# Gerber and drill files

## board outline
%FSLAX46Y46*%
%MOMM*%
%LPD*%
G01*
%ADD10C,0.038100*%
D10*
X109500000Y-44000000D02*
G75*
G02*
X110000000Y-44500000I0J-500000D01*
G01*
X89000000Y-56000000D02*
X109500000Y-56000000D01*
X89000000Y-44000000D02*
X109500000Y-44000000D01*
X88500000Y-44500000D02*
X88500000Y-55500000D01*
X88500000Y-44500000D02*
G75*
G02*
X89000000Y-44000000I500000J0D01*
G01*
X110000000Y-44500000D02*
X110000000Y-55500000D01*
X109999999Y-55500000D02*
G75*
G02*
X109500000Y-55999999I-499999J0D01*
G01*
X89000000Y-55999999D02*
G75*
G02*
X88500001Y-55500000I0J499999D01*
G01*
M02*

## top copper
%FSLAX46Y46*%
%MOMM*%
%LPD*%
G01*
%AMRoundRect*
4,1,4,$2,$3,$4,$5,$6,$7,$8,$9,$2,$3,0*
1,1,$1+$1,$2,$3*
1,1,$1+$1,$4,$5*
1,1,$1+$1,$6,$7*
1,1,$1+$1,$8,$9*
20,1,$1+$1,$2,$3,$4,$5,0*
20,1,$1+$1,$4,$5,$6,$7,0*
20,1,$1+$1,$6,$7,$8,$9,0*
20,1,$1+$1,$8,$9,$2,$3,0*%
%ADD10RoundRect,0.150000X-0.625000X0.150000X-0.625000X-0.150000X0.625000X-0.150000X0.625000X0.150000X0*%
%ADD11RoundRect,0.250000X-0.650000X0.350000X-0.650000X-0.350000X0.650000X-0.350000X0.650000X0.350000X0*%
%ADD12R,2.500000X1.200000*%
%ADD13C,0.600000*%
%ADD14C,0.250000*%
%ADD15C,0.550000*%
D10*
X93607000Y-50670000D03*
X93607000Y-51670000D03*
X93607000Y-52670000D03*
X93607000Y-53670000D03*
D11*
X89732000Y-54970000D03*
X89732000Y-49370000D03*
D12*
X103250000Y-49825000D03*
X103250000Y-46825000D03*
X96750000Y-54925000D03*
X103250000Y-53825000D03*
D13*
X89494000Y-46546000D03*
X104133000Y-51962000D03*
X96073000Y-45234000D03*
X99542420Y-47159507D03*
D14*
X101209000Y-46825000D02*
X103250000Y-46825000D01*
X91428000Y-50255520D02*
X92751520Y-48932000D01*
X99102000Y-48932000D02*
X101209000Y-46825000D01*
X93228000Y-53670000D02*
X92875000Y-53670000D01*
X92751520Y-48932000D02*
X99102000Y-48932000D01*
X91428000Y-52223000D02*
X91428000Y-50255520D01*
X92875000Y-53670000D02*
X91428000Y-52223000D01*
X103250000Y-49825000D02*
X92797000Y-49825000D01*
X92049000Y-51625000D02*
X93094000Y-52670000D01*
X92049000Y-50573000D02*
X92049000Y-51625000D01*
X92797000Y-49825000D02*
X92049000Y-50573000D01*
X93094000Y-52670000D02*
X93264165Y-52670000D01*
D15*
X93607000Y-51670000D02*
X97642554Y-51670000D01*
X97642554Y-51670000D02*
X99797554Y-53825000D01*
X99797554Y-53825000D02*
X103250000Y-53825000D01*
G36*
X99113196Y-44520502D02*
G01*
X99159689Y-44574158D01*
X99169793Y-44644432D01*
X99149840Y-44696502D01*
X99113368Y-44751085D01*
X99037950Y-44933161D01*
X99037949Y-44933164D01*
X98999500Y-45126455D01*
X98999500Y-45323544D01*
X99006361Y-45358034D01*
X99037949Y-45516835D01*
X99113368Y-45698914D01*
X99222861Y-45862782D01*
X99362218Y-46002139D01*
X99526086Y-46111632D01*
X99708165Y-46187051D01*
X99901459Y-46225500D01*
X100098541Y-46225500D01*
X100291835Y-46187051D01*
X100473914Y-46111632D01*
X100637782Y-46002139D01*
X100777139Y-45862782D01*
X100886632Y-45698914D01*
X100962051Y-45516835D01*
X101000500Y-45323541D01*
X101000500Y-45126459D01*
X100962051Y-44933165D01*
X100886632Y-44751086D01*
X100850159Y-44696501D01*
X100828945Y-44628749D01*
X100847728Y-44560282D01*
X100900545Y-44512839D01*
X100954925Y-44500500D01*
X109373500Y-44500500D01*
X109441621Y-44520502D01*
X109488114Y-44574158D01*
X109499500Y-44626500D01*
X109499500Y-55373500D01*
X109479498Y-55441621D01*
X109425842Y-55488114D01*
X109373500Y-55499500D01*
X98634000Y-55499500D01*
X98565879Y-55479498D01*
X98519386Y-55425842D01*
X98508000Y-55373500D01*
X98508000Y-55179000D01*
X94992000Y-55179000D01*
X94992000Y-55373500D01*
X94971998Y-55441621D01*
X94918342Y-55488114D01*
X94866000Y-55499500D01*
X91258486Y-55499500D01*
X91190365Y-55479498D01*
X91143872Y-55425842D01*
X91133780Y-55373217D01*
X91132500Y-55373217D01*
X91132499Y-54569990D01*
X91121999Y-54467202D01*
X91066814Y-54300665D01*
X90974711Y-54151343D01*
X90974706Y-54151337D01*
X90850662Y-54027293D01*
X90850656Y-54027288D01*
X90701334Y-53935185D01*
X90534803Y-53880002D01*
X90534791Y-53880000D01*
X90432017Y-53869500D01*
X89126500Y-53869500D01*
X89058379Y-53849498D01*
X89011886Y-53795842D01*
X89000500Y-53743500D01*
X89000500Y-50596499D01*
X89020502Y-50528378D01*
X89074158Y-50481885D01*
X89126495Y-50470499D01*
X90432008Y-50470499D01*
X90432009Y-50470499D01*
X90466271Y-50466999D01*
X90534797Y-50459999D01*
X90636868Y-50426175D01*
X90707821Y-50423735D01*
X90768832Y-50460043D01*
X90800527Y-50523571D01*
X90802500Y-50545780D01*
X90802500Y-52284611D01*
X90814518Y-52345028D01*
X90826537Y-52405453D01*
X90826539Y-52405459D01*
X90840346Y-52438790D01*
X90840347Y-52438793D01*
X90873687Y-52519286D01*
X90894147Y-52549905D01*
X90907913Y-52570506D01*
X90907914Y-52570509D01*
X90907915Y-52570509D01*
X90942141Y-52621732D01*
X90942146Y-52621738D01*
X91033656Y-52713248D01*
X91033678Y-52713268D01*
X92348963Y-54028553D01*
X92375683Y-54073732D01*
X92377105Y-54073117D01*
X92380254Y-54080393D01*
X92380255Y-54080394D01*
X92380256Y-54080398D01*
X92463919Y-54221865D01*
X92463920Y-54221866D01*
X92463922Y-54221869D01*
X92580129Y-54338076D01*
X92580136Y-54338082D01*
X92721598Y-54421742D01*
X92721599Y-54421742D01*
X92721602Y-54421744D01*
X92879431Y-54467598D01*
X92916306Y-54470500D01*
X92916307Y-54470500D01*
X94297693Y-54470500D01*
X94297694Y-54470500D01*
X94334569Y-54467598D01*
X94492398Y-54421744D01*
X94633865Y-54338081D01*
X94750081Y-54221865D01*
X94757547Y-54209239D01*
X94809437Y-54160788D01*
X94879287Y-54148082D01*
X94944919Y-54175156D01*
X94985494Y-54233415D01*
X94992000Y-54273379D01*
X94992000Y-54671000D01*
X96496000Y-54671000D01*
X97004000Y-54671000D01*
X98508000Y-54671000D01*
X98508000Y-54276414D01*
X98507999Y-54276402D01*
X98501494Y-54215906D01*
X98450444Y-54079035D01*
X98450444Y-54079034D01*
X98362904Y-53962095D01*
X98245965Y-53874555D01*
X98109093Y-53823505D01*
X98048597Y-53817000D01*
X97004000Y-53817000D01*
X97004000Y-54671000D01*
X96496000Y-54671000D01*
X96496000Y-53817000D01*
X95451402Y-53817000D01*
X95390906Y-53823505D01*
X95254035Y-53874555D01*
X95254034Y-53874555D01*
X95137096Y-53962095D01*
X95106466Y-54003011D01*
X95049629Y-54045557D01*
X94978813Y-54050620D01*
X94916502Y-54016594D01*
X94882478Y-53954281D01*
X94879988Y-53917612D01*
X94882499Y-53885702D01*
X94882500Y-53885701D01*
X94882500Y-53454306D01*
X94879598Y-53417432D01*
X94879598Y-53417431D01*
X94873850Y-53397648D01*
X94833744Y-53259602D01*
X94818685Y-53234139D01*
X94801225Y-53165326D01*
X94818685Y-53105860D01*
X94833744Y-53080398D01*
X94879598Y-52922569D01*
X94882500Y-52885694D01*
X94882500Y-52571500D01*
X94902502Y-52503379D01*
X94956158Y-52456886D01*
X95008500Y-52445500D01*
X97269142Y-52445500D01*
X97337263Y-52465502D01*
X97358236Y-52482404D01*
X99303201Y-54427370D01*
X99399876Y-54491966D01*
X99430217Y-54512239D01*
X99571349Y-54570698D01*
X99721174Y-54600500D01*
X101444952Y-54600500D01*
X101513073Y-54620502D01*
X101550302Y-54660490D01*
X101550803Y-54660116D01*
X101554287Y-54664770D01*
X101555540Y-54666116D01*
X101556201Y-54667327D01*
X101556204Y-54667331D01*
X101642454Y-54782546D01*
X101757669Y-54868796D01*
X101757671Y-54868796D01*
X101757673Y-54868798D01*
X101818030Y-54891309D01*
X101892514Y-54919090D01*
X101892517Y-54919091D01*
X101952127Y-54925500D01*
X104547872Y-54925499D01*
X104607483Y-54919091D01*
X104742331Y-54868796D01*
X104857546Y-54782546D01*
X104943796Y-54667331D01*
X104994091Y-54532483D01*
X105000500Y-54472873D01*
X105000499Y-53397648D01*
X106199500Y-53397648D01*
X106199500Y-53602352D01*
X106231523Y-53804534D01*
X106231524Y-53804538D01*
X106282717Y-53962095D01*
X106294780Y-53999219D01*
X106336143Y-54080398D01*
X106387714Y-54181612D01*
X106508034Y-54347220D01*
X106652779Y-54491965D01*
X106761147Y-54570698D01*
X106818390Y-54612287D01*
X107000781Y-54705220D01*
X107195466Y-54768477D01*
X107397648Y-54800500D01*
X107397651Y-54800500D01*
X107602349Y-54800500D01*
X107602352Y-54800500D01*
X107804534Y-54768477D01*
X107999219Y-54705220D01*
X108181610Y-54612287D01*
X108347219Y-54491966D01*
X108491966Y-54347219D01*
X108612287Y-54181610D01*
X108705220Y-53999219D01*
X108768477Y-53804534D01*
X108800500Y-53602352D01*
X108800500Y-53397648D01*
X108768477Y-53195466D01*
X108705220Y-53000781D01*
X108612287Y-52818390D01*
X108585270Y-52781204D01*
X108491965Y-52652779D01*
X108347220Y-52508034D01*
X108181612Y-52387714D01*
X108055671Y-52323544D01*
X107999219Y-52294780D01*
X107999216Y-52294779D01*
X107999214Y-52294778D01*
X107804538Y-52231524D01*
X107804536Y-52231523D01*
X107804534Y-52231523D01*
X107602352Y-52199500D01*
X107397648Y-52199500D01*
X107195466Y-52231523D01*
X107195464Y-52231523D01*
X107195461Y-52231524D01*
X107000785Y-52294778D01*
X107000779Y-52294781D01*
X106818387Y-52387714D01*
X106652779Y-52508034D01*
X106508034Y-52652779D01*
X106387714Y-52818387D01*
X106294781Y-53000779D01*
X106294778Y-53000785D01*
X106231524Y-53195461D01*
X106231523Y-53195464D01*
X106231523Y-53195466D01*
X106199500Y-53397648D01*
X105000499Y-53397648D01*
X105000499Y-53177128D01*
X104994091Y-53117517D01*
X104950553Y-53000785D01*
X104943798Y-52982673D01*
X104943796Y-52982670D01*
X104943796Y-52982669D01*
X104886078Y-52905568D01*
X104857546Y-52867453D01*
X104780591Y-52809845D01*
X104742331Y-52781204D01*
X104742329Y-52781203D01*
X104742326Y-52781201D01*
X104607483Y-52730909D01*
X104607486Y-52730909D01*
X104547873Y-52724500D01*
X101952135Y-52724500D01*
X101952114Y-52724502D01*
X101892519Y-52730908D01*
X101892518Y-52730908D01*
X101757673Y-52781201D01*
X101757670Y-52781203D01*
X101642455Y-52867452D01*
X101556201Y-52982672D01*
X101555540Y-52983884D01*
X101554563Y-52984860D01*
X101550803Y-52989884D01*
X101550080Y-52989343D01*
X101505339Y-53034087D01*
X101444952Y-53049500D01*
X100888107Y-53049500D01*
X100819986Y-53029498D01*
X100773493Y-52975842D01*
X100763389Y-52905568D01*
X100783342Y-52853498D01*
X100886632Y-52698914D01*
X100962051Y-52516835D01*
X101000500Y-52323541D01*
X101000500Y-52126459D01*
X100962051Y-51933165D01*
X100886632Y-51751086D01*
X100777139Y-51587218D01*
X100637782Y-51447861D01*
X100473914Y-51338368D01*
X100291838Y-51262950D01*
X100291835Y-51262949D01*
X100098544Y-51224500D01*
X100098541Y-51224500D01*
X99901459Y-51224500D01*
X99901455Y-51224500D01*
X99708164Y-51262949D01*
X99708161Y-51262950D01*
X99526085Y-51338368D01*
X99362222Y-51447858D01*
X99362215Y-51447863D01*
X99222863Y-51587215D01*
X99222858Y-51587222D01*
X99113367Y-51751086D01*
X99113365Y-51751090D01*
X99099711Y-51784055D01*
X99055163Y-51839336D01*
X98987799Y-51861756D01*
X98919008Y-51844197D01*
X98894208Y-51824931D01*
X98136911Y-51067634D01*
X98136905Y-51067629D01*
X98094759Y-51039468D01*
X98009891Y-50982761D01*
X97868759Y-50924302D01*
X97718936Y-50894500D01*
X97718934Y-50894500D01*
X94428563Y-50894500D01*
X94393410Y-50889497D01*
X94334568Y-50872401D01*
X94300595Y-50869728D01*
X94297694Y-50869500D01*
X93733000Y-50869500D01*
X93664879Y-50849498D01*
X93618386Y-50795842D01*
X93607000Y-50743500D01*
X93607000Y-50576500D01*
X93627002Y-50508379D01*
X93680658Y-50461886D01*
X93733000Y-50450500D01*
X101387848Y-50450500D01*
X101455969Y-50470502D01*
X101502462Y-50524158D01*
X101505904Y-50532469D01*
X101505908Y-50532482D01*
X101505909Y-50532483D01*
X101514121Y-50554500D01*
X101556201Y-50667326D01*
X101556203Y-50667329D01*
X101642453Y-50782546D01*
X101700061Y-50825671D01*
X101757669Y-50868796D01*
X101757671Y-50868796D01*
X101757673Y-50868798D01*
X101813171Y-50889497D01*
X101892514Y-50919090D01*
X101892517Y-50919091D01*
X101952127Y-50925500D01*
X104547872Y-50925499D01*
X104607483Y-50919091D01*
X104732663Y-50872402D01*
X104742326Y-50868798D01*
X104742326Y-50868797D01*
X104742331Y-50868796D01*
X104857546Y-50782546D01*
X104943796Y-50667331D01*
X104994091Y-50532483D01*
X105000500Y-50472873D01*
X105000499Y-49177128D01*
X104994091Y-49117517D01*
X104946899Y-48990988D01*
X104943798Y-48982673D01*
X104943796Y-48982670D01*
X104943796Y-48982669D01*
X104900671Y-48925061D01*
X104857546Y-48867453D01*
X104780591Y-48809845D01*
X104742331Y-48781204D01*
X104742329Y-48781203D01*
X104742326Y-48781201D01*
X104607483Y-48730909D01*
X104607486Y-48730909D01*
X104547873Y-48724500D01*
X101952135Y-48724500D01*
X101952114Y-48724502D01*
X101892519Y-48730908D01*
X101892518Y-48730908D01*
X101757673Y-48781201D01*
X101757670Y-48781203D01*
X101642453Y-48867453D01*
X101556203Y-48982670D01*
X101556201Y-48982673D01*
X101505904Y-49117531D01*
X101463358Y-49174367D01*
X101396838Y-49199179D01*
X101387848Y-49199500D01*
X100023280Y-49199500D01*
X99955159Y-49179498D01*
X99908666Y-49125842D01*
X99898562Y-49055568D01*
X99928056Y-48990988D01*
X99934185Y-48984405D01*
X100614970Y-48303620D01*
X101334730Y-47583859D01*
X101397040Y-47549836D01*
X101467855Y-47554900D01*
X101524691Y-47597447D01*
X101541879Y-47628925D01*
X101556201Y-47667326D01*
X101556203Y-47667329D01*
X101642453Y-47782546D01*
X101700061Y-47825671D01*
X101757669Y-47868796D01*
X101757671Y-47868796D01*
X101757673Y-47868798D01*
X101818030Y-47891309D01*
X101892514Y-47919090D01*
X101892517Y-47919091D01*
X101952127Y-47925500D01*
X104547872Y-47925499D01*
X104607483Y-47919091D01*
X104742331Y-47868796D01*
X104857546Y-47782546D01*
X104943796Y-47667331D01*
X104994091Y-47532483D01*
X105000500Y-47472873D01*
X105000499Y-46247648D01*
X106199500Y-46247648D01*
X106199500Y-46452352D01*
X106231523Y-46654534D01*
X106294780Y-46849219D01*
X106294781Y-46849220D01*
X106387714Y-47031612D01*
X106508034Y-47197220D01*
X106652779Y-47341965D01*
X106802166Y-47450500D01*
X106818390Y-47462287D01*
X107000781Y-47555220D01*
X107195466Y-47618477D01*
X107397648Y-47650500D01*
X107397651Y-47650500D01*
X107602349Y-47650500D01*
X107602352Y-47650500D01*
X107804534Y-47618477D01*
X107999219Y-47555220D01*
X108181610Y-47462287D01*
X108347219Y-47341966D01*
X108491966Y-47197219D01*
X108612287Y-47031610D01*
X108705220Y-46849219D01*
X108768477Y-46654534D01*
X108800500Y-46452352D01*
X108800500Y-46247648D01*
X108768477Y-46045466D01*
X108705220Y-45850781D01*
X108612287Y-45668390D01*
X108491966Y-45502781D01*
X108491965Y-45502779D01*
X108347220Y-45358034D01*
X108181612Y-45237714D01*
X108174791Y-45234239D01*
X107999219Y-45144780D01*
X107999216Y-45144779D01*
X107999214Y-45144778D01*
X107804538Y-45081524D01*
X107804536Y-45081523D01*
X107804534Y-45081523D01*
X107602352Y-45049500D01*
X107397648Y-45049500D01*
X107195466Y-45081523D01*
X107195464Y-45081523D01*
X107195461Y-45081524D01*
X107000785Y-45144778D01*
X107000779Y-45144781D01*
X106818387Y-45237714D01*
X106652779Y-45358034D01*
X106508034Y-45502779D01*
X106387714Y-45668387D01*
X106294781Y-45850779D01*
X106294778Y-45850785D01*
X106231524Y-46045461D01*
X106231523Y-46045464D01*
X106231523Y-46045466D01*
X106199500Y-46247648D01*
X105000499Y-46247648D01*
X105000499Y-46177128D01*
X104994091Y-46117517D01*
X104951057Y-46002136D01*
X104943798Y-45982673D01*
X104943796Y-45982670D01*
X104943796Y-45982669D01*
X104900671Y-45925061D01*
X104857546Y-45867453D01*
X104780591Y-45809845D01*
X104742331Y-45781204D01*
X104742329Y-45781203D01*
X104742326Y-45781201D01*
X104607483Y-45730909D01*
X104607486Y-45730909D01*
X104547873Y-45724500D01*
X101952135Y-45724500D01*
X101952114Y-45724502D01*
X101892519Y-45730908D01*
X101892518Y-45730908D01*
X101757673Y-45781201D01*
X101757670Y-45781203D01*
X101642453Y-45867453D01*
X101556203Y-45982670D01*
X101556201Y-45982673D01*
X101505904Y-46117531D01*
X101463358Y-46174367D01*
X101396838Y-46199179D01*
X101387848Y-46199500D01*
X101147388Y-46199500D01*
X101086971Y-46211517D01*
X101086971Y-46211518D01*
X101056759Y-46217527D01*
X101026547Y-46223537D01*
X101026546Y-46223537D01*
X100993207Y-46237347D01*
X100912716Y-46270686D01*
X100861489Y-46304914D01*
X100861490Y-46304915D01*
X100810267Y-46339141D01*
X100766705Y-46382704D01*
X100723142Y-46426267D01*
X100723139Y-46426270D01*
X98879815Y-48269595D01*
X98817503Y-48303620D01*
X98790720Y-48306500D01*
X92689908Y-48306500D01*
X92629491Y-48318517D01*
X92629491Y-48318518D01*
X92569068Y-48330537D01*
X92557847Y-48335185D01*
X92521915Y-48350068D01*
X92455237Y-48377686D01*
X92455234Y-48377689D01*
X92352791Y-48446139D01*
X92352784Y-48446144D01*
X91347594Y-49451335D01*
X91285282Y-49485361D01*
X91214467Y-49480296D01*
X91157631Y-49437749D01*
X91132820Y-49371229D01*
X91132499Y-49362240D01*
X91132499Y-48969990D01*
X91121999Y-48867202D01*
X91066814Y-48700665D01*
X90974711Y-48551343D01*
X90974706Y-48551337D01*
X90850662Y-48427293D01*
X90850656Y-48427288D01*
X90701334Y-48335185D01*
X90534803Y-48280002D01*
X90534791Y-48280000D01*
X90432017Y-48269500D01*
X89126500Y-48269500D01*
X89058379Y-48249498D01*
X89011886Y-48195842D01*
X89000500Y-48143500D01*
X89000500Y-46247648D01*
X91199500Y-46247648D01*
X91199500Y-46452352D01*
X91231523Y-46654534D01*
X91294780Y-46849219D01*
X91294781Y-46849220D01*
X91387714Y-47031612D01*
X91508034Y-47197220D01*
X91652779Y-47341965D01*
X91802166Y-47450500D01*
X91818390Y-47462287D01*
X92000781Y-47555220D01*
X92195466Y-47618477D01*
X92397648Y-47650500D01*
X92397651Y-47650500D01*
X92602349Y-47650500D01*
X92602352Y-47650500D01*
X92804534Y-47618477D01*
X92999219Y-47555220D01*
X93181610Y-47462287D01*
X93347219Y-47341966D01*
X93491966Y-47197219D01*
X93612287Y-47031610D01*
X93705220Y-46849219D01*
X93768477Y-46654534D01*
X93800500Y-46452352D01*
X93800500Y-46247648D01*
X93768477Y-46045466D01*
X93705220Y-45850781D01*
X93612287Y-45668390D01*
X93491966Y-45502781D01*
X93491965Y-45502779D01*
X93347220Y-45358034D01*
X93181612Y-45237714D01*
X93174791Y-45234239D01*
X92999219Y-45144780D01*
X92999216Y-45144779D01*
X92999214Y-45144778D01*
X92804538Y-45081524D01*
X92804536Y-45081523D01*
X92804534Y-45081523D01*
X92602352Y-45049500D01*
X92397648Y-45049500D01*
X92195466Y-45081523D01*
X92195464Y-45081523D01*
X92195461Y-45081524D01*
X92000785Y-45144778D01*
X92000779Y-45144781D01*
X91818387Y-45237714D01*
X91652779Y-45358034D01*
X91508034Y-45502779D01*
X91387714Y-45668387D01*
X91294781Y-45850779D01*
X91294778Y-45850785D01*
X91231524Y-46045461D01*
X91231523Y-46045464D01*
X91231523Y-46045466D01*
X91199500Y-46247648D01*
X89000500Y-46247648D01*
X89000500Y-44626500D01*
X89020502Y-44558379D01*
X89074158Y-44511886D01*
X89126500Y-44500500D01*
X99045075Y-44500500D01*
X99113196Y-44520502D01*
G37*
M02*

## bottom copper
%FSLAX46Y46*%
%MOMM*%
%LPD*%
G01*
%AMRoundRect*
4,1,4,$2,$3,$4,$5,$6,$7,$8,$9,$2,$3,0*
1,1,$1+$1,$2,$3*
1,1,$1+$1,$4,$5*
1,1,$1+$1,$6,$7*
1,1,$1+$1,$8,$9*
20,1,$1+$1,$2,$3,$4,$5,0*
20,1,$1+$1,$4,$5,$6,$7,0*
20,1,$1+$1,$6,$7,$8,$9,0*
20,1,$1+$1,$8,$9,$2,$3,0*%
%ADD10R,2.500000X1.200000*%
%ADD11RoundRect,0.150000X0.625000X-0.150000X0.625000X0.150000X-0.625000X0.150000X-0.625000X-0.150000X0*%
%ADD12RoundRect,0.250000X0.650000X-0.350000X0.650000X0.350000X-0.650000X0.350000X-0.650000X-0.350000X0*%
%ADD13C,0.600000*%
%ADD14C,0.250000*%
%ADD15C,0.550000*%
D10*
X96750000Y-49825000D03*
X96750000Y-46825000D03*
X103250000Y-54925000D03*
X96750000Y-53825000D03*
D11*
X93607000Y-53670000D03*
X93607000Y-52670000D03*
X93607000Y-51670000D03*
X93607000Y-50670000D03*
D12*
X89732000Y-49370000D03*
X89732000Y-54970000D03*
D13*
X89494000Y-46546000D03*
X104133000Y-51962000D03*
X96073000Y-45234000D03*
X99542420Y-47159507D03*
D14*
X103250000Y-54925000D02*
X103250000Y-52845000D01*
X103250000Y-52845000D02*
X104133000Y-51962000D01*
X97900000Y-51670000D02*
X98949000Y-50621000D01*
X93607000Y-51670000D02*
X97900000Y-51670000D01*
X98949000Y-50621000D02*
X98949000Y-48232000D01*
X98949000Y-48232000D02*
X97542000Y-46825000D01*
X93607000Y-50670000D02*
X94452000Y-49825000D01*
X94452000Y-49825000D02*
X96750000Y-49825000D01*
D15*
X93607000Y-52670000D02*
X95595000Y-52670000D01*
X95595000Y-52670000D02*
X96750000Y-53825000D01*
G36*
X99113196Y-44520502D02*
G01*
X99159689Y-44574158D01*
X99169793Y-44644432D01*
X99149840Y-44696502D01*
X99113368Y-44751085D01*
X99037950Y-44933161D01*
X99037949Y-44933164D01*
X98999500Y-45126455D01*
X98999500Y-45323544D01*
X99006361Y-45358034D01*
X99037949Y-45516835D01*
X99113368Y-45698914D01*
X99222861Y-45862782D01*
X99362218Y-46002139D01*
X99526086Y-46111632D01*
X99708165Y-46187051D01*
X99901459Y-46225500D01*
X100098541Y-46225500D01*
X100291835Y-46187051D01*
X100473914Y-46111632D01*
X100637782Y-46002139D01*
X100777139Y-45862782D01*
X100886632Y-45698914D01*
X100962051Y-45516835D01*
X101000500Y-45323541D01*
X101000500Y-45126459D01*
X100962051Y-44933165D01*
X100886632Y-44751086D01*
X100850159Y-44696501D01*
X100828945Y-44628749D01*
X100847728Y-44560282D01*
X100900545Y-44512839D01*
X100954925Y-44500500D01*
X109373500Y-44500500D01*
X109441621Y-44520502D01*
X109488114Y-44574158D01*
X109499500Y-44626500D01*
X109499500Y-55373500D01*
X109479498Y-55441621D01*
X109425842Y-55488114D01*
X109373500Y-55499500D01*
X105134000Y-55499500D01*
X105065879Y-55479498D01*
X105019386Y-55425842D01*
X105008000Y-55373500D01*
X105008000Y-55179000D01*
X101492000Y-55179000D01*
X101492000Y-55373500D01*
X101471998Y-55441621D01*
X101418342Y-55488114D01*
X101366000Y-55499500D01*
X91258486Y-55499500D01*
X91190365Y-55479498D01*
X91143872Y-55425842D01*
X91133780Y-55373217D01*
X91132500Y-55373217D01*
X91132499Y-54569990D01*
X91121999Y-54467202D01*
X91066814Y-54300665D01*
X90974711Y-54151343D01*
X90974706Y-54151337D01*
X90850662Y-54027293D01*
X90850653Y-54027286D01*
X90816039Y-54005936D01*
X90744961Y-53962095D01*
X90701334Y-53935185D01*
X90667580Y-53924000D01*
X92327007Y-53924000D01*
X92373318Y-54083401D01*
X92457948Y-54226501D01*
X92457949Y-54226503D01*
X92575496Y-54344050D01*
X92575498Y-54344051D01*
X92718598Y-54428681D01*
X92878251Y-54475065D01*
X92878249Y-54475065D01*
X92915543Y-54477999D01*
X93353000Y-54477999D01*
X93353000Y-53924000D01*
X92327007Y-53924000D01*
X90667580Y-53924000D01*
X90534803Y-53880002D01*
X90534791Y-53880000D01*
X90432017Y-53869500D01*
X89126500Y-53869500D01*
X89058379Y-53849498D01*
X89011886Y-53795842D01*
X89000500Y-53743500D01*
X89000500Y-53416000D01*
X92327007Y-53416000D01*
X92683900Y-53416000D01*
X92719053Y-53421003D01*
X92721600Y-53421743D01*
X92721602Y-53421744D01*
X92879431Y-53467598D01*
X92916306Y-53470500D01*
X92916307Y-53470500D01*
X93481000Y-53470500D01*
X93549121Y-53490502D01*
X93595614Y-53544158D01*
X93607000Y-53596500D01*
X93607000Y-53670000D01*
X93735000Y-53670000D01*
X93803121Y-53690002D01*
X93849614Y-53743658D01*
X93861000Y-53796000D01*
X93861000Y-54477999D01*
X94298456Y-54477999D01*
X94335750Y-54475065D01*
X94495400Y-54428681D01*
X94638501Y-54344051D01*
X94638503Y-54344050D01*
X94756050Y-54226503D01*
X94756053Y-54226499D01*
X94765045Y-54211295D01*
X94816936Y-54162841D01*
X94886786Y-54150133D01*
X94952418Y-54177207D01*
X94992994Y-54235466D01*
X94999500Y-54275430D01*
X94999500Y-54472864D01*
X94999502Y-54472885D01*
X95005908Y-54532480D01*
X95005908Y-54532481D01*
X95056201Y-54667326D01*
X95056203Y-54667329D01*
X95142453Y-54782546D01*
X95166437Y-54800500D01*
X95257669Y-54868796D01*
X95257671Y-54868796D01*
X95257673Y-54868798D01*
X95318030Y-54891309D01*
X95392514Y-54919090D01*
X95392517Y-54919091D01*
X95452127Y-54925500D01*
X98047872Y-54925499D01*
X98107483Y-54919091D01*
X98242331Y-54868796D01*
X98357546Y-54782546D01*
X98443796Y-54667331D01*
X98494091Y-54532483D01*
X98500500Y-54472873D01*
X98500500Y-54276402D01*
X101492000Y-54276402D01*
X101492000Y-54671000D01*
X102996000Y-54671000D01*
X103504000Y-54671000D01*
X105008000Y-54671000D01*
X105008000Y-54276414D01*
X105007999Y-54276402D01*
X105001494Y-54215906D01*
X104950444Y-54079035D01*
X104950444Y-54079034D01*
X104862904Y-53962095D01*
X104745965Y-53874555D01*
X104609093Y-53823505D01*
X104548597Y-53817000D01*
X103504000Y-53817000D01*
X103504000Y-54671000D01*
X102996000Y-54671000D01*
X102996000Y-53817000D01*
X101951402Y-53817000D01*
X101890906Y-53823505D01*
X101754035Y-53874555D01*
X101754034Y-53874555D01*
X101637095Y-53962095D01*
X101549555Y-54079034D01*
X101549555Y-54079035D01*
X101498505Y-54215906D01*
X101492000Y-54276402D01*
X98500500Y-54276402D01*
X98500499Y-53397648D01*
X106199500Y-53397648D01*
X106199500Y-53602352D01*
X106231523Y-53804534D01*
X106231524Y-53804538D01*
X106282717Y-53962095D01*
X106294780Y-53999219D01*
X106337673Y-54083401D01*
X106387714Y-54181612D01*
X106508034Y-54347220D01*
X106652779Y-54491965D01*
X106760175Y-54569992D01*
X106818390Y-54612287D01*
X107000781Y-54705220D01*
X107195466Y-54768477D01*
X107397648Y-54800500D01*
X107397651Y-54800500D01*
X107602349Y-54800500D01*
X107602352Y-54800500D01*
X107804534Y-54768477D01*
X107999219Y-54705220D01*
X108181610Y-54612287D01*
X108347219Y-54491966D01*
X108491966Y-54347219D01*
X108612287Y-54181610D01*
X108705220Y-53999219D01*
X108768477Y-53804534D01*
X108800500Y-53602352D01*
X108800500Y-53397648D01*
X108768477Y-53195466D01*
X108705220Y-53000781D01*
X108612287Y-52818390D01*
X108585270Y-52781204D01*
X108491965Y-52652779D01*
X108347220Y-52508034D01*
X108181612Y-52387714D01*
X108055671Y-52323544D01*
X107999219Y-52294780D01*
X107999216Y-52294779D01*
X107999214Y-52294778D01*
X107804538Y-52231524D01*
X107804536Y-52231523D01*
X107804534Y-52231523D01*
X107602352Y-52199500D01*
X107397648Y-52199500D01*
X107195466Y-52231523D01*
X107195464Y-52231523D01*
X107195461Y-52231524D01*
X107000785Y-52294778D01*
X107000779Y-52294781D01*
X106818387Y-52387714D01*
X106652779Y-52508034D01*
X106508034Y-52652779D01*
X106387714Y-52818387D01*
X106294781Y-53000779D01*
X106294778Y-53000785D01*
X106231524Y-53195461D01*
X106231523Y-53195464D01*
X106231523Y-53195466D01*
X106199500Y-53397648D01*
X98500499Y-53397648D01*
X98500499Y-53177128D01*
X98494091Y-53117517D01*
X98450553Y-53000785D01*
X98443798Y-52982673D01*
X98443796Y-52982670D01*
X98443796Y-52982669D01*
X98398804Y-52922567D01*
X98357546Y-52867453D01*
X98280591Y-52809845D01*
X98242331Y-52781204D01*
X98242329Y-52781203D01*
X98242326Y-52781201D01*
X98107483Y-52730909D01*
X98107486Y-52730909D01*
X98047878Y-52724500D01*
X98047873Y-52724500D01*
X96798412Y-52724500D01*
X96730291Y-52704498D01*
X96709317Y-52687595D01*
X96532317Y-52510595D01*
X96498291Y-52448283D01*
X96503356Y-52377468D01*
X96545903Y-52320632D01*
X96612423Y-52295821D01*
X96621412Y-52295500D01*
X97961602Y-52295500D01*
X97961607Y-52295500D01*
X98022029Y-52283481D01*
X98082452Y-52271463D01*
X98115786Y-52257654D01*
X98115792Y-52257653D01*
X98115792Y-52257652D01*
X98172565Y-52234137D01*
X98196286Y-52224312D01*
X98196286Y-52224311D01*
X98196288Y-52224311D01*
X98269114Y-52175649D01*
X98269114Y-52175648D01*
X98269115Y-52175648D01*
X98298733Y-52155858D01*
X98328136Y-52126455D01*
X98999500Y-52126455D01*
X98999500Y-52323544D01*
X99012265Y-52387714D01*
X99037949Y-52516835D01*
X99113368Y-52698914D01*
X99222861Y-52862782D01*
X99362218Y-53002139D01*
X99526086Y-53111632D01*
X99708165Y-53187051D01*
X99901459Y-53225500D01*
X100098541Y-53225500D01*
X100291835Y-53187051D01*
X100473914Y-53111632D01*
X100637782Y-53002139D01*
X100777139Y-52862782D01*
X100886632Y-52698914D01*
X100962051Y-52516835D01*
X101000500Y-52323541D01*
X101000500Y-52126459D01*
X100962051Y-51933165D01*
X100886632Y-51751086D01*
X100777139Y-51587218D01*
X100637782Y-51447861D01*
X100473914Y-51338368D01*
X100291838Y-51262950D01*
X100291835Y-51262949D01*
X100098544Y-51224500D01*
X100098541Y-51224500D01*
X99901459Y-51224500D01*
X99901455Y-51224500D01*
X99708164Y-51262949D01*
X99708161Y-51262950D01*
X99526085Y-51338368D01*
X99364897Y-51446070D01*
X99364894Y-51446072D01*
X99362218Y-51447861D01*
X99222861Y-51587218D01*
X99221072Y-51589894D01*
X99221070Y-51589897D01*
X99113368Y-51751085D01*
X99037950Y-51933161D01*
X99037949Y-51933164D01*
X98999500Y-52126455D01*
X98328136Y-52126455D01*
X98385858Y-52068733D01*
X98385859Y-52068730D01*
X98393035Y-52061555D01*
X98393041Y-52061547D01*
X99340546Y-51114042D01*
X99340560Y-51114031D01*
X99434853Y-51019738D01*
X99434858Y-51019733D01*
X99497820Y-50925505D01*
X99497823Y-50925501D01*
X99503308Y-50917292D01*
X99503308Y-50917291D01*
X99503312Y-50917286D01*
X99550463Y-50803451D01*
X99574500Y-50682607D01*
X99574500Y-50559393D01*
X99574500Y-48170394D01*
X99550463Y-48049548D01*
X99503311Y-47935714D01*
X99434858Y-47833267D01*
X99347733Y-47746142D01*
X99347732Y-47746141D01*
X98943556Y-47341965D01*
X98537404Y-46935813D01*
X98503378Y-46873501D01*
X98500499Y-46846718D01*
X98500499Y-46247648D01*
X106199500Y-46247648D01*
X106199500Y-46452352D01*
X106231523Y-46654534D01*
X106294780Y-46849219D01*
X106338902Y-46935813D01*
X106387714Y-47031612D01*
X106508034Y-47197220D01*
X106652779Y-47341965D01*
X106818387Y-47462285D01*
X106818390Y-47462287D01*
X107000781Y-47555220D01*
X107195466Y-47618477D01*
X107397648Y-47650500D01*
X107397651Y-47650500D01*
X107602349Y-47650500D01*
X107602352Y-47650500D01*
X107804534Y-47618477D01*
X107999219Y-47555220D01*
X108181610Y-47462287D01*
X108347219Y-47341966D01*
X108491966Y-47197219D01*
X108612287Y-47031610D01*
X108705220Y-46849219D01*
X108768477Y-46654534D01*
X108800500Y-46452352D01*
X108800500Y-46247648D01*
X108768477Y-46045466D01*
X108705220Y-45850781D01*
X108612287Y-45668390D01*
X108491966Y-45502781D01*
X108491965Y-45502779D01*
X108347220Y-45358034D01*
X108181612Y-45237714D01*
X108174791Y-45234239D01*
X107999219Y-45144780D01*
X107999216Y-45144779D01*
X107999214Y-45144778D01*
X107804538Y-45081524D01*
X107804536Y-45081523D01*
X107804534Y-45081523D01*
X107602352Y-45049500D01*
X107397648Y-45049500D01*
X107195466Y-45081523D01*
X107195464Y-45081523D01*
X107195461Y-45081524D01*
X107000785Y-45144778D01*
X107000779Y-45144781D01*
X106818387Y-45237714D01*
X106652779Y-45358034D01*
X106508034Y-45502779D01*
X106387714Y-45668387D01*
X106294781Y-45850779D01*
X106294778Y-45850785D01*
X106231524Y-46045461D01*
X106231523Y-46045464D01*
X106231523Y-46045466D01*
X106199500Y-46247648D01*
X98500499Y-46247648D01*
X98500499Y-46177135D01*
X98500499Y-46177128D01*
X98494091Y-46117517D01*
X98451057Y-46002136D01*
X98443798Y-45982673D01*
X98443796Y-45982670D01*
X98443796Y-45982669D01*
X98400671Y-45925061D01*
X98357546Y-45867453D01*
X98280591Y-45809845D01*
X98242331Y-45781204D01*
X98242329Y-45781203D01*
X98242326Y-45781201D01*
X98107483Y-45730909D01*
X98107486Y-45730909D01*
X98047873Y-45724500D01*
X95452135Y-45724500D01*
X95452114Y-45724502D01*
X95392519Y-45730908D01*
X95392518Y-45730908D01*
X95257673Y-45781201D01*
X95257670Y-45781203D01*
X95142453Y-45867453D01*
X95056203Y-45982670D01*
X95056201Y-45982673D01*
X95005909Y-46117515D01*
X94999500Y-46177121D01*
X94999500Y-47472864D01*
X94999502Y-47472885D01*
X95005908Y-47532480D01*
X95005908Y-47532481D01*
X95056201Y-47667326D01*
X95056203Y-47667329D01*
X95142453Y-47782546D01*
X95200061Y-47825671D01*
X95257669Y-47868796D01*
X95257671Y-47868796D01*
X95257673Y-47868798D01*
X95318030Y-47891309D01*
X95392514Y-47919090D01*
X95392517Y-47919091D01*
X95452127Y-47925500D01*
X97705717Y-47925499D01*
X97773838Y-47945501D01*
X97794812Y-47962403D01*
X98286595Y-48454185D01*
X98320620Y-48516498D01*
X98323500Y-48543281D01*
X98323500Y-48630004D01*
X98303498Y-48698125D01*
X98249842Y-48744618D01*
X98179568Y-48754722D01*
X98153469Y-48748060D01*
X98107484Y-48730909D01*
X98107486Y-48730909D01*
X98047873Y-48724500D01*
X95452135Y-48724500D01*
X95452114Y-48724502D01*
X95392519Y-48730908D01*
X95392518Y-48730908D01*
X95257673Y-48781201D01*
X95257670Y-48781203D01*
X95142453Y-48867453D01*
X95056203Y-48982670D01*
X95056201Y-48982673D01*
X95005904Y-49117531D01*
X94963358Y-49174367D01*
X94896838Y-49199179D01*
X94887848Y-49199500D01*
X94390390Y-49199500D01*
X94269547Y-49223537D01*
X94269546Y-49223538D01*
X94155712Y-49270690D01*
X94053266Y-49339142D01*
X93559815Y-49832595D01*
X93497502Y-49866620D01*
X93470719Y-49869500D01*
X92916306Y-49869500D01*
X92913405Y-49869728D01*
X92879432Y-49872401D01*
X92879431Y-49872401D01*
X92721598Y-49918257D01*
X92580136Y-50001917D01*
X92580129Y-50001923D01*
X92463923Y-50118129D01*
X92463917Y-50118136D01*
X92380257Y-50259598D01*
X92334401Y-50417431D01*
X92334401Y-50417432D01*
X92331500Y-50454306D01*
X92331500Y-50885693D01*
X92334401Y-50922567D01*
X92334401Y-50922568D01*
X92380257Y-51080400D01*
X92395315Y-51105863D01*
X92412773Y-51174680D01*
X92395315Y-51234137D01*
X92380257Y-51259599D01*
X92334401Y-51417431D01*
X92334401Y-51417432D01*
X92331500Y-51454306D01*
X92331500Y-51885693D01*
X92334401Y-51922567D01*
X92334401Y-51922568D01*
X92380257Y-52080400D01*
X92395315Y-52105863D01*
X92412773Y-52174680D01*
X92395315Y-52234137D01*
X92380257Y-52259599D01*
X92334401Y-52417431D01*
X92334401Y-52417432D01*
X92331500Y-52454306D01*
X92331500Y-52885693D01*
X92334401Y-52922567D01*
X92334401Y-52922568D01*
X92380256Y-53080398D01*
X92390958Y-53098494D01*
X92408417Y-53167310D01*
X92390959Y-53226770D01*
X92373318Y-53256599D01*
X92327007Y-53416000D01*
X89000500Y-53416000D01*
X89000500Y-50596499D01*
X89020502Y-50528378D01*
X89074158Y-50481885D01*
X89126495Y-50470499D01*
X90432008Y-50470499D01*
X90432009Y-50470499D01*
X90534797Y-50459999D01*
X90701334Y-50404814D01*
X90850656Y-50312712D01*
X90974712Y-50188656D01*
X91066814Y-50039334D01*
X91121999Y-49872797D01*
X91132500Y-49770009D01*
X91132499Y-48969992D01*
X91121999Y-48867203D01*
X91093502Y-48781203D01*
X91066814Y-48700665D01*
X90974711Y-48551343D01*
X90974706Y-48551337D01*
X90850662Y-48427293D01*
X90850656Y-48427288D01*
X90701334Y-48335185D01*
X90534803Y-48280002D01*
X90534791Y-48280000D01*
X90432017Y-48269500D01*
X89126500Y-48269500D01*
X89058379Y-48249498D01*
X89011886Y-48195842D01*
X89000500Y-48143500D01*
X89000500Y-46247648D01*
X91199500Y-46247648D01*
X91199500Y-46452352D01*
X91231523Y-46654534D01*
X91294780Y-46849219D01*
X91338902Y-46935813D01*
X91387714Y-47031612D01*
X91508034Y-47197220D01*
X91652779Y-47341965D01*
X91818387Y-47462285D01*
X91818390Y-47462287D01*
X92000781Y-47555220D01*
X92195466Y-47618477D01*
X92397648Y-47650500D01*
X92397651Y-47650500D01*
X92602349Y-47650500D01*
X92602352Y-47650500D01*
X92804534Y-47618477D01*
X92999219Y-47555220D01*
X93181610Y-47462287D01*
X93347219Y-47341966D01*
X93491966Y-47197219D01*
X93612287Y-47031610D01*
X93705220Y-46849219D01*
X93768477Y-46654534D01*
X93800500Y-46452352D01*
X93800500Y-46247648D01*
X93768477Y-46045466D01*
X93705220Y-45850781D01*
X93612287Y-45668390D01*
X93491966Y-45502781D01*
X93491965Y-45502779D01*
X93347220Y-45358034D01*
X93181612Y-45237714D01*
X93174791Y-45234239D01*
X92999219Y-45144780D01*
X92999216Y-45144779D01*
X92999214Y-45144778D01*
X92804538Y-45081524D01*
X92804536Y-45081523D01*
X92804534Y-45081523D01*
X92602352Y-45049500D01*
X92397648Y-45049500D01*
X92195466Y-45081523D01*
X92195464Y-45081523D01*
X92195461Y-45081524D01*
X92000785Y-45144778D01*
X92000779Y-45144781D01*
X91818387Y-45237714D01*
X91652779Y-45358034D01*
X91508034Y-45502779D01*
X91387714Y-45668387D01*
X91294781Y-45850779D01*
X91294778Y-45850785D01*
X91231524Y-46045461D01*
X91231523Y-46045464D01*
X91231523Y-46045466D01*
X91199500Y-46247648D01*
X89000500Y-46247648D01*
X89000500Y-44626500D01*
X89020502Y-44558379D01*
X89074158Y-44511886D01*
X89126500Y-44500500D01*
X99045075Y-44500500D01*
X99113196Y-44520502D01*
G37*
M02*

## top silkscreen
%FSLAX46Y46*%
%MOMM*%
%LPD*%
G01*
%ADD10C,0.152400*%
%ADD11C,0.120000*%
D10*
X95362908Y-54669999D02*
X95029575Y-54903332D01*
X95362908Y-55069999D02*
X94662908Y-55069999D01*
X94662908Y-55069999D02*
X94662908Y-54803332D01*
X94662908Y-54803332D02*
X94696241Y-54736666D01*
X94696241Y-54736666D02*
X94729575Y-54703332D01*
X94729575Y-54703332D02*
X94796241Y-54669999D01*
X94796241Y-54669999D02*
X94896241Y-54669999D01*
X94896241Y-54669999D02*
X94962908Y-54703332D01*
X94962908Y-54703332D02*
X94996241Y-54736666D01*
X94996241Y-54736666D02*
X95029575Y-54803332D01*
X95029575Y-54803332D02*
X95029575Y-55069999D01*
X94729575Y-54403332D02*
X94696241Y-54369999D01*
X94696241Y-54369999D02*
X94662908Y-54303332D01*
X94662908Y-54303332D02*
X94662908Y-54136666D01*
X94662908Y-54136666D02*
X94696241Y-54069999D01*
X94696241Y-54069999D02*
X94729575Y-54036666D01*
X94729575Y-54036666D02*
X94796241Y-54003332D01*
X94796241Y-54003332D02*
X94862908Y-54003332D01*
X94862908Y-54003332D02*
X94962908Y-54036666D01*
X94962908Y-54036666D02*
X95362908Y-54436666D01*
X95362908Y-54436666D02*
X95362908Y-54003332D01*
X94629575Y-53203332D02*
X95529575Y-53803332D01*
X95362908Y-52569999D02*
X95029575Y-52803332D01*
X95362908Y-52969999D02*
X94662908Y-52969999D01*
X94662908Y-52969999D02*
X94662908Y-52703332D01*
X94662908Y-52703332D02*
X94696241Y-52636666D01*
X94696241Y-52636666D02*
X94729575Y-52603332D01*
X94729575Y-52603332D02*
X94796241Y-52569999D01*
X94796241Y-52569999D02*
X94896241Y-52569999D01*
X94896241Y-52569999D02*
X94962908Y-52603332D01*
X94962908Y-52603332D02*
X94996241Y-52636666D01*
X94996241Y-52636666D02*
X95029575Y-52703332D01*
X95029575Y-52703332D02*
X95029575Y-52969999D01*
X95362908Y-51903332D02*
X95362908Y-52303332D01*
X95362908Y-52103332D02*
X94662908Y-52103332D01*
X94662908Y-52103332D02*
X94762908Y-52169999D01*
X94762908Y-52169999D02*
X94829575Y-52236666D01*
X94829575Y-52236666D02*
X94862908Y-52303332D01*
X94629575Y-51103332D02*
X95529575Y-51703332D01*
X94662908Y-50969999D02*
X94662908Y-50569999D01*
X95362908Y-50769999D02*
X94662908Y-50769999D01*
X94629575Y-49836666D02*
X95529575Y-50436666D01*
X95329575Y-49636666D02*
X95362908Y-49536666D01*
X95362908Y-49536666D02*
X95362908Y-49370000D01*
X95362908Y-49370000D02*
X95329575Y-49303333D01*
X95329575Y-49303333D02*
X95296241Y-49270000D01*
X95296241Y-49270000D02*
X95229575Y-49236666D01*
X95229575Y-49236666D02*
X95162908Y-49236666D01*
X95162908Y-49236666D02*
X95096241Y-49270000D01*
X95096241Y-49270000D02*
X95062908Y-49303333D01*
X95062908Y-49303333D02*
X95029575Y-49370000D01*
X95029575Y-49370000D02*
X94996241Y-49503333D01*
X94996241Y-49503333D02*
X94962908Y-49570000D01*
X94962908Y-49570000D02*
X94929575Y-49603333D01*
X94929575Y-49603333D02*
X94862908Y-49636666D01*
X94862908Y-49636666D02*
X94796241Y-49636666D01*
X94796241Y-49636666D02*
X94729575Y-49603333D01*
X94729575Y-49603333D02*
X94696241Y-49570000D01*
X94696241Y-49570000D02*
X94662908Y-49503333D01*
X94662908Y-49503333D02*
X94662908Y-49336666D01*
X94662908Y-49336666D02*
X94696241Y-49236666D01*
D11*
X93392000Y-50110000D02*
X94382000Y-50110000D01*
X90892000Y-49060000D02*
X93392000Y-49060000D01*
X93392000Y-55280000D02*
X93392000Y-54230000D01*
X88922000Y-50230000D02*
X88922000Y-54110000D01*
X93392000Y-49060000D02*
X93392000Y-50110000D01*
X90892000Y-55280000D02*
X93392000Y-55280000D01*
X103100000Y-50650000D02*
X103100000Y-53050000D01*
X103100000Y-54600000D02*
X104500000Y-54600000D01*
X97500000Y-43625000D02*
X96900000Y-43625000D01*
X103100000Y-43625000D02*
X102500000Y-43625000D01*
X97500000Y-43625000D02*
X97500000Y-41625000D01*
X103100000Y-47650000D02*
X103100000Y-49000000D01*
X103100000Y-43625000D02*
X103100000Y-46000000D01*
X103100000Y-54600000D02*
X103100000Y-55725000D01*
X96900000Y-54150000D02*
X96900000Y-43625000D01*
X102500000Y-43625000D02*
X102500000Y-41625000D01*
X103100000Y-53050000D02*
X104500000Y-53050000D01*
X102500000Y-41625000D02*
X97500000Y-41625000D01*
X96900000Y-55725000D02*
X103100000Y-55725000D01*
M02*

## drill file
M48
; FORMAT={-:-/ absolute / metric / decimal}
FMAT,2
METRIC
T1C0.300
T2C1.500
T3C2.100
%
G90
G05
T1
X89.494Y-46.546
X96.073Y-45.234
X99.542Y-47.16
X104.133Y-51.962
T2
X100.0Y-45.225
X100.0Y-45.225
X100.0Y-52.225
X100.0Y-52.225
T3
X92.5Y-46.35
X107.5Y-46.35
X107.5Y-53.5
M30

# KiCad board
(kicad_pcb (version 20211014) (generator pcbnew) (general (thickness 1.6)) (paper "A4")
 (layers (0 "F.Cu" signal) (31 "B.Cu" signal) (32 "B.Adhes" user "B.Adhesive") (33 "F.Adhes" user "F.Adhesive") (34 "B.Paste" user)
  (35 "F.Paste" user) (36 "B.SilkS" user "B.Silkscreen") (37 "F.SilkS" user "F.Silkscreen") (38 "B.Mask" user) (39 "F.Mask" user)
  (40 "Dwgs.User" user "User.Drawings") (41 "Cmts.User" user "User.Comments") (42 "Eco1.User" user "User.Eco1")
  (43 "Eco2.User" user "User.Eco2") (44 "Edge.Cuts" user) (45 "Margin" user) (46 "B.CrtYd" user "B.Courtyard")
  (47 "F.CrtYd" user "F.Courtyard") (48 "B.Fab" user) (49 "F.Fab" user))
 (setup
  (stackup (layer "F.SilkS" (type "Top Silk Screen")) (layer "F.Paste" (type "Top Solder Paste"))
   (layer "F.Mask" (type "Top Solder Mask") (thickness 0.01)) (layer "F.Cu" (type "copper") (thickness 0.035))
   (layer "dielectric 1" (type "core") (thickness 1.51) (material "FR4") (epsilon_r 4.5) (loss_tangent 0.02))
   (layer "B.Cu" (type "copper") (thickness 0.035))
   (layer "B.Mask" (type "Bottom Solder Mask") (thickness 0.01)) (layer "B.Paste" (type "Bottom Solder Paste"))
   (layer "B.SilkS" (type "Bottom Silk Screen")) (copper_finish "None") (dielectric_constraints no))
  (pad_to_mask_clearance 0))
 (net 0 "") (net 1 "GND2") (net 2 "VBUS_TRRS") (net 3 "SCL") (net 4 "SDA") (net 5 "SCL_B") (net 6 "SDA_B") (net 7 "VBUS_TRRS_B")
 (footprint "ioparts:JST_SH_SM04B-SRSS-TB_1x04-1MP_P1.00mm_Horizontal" (layer "F.Cu") (at 91.607 52.17 -90)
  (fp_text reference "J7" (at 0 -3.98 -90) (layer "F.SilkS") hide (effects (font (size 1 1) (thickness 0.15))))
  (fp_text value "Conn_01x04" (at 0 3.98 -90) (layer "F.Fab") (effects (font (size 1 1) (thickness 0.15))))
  (fp_line (start -2.06 -1.785) (end -2.06 -2.775) (layer "F.SilkS") (width 0.12))
  (fp_line (start -3.11 0.715) (end -3.11 -1.785) (layer "F.SilkS") (width 0.12))
  (fp_line (start 3.11 -1.785) (end 2.06 -1.785) (layer "F.SilkS") (width 0.12))
  (fp_line (start -1.94 2.685) (end 1.94 2.685) (layer "F.SilkS") (width 0.12))
  (fp_line (start -3.11 -1.785) (end -2.06 -1.785) (layer "F.SilkS") (width 0.12))
  (fp_line (start 3.11 0.715) (end 3.11 -1.785) (layer "F.SilkS") (width 0.12))
  (pad "1" smd roundrect (at -1.5 -2 270) (size 0.6 1.55) (layers "F.Cu" "F.Paste" "F.Mask") (roundrect_rratio 0.25) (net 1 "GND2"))
  (pad "2" smd roundrect (at -0.5 -2 270) (size 0.6 1.55) (layers "F.Cu" "F.Paste" "F.Mask") (roundrect_rratio 0.25) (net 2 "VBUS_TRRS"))
  (pad "3" smd roundrect (at 0.5 -2 270) (size 0.6 1.55) (layers "F.Cu" "F.Paste" "F.Mask") (roundrect_rratio 0.25) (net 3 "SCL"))
  (pad "4" smd roundrect (at 1.5 -2 270) (size 0.6 1.55) (layers "F.Cu" "F.Paste" "F.Mask") (roundrect_rratio 0.25) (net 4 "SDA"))
  (pad "MP" smd roundrect (at 2.8 1.875 270) (size 1.2 1.8) (layers "F.Cu" "F.Paste" "F.Mask") (roundrect_rratio 0.2083333333))
  (pad "MP" smd roundrect (at -2.8 1.875 270) (size 1.2 1.8) (layers "F.Cu" "F.Paste" "F.Mask") (roundrect_rratio 0.2083333333)))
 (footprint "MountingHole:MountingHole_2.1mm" (layer "F.Cu") (at 107.5 53.5)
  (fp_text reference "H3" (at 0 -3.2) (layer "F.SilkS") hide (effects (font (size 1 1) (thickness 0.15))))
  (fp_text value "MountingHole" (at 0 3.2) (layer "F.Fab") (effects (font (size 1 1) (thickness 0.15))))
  (pad "" np_thru_hole circle (at 0 0) (size 2.1 2.1) (drill 2.1) (layers *.Cu *.Mask)))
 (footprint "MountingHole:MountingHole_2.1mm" (layer "F.Cu") (at 92.5 46.35)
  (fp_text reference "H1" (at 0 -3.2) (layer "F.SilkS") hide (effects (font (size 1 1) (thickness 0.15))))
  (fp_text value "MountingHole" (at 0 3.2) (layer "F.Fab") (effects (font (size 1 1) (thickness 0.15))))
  (pad "" np_thru_hole circle (at 0 0) (size 2.1 2.1) (drill 2.1) (layers *.Cu *.Mask)))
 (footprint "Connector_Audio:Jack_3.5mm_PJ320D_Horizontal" (layer "F.Cu") (at 100 50 -90)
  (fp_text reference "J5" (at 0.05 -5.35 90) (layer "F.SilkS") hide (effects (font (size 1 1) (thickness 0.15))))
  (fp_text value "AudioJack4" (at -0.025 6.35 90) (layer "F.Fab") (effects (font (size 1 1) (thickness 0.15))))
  (fp_line (start 0.65 -3.1) (end 3.05 -3.1) (layer "F.SilkS") (width 0.12))
  (fp_line (start 4.6 -3.1) (end 4.6 -4.5) (layer "F.SilkS") (width 0.12))
  (fp_line (start -6.375 2.5) (end -6.375 3.1) (layer "F.SilkS") (width 0.12))
  (fp_line (start -6.375 -3.1) (end -6.375 -2.5) (layer "F.SilkS") (width 0.12))
  (fp_line (start -6.375 2.5) (end -8.375 2.5) (layer "F.SilkS") (width 0.12))
  (fp_line (start -2.35 -3.1) (end -1 -3.1) (layer "F.SilkS") (width 0.12))
  (fp_line (start -6.375 -3.1) (end -4 -3.1) (layer "F.SilkS") (width 0.12))
  (fp_line (start 4.6 -3.1) (end 5.725 -3.1) (layer "F.SilkS") (width 0.12))
  (fp_line (start 4.15 3.1) (end -6.375 3.1) (layer "F.SilkS") (width 0.12))
  (fp_line (start -6.375 -2.5) (end -8.375 -2.5) (layer "F.SilkS") (width 0.12))
  (fp_line (start 3.05 -3.1) (end 3.05 -4.5) (layer "F.SilkS") (width 0.12))
  (fp_line (start -8.375 -2.5) (end -8.375 2.5) (layer "F.SilkS") (width 0.12))
  (fp_line (start 5.725 3.1) (end 5.725 -3.1) (layer "F.SilkS") (width 0.12))
  (pad "" np_thru_hole circle (at -4.775 0 270) (size 1.5 1.5) (drill 1.5) (layers *.Cu *.Mask))
  (pad "" np_thru_hole circle (at 2.225 0 270) (size 1.5 1.5) (drill 1.5) (layers *.Cu *.Mask))
  (pad "R1" smd rect (at -0.175 -3.25 270) (size 1.2 2.5) (layers "F.Cu" "F.Paste" "F.Mask") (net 3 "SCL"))
  (pad "R2" smd rect (at -3.175 -3.25 270) (size 1.2 2.5) (layers "F.Cu" "F.Paste" "F.Mask") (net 4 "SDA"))
  (pad "S" smd rect (at 4.925 3.25 270) (size 1.2 2.5) (layers "F.Cu" "F.Paste" "F.Mask") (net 1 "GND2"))
  (pad "T" smd rect (at 3.825 -3.25 270) (size 1.2 2.5) (layers "F.Cu" "F.Paste" "F.Mask") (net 2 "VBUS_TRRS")))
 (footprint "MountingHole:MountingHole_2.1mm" (layer "F.Cu") (at 107.5 46.35)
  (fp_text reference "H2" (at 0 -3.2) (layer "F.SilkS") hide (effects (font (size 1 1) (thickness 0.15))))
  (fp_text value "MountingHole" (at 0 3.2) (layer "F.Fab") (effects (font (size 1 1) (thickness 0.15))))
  (pad "" np_thru_hole circle (at 0 0) (size 2.1 2.1) (drill 2.1) (layers *.Cu *.Mask)))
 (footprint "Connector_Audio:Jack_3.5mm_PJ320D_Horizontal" (layer "B.Cu") (at 100 50 -90)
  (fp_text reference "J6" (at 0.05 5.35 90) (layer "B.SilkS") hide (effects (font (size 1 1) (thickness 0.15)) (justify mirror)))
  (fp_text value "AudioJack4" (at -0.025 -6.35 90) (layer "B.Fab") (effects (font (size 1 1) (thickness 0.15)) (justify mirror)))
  (pad "" np_thru_hole circle (at 2.225 0 270) (size 1.5 1.5) (drill 1.5) (layers *.Cu *.Mask))
  (pad "" np_thru_hole circle (at -4.775 0 270) (size 1.5 1.5) (drill 1.5) (layers *.Cu *.Mask))
  (pad "R1" smd rect (at -0.175 3.25 270) (size 1.2 2.5) (layers "B.Cu" "B.Paste" "B.Mask") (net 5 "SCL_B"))
  (pad "R2" smd rect (at -3.175 3.25 270) (size 1.2 2.5) (layers "B.Cu" "B.Paste" "B.Mask") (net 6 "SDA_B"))
  (pad "S" smd rect (at 4.925 -3.25 270) (size 1.2 2.5) (layers "B.Cu" "B.Paste" "B.Mask") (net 1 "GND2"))
  (pad "T" smd rect (at 3.825 3.25 270) (size 1.2 2.5) (layers "B.Cu" "B.Paste" "B.Mask") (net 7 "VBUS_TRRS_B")))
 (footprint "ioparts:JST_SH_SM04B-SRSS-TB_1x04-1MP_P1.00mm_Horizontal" (layer "B.Cu") (at 91.607 52.17 90)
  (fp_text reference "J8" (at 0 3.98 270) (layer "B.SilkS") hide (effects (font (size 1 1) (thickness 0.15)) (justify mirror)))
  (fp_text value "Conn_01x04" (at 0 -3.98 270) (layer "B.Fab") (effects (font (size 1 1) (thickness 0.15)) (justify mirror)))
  (pad "1" smd roundrect (at -1.5 2 90) (size 0.6 1.55) (layers "B.Cu" "B.Paste" "B.Mask") (roundrect_rratio 0.25) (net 1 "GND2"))
  (pad "2" smd roundrect (at -0.5 2 90) (size 0.6 1.55) (layers "B.Cu" "B.Paste" "B.Mask") (roundrect_rratio 0.25) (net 7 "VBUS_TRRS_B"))
  (pad "3" smd roundrect (at 0.5 2 90) (size 0.6 1.55) (layers "B.Cu" "B.Paste" "B.Mask") (roundrect_rratio 0.25) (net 6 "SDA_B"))
  (pad "4" smd roundrect (at 1.5 2 90) (size 0.6 1.55) (layers "B.Cu" "B.Paste" "B.Mask") (roundrect_rratio 0.25) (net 5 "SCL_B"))
  (pad "MP" smd roundrect (at 2.8 -1.875 90) (size 1.2 1.8) (layers "B.Cu" "B.Paste" "B.Mask") (roundrect_rratio 0.2083333333))
  (pad "MP" smd roundrect (at -2.8 -1.875 90) (size 1.2 1.8) (layers "B.Cu" "B.Paste" "B.Mask") (roundrect_rratio 0.2083333333)))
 (gr_arc (start 109.5 44) (mid 109.853553 44.146447) (end 110 44.5) (layer "Edge.Cuts") (width 0.0381))
 (gr_line (start 89 56) (end 109.5 56) (layer "Edge.Cuts") (width 0.0381))
 (gr_line (start 89 44) (end 109.5 44) (layer "Edge.Cuts") (width 0.0381))
 (gr_line (start 88.5 44.5) (end 88.5 55.5) (layer "Edge.Cuts") (width 0.0381))
 (gr_arc (start 88.5 44.5) (mid 88.646447 44.146447) (end 89 44.000001) (layer "Edge.Cuts") (width 0.0381))
 (gr_line (start 110 44.5) (end 110 55.5) (layer "Edge.Cuts") (width 0.0381))
 (gr_arc (start 109.999999 55.5) (mid 109.853553 55.853553) (end 109.5 55.999999) (layer "Edge.Cuts") (width 0.0381))
 (gr_arc (start 89 55.999999) (mid 88.646447 55.853553) (end 88.5 55.5) (layer "Edge.Cuts") (width 0.0381))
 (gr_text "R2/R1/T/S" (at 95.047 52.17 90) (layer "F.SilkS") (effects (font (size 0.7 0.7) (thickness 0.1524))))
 (segment (start 101.209 46.825) (end 103.25 46.825) (width 0.25) (layer "F.Cu") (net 4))
 (segment (start 91.428 50.25552) (end 92.75152 48.932) (width 0.25) (layer "F.Cu") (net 4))
 (segment (start 99.102 48.932) (end 101.209 46.825) (width 0.25) (layer "F.Cu") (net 4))
 (segment (start 93.228 53.67) (end 92.875 53.67) (width 0.25) (layer "F.Cu") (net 4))
 (segment (start 92.75152 48.932) (end 99.102 48.932) (width 0.25) (layer "F.Cu") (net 4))
 (segment (start 91.428 52.223) (end 91.428 50.25552) (width 0.25) (layer "F.Cu") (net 4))
 (segment (start 92.875 53.67) (end 91.428 52.223) (width 0.25) (layer "F.Cu") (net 4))
 (segment (start 103.25 49.825) (end 92.797 49.825) (width 0.25) (layer "F.Cu") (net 3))
 (segment (start 92.049 51.625) (end 93.094 52.67) (width 0.25) (layer "F.Cu") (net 3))
 (segment (start 92.049 50.573) (end 92.049 51.625) (width 0.25) (layer "F.Cu") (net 3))
 (segment (start 92.797 49.825) (end 92.049 50.573) (width 0.25) (layer "F.Cu") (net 3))
 (segment (start 93.094 52.67) (end 93.264165 52.67) (width 0.25) (layer "F.Cu") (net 3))
 (via (at 89.494 46.546) (size 0.6) (drill 0.3) (layers "F.Cu" "B.Cu") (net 1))
 (via (at 104.133 51.962) (size 0.6) (drill 0.3) (layers "F.Cu" "B.Cu") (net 1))
 (via (at 96.073 45.234) (size 0.6) (drill 0.3) (layers "F.Cu" "B.Cu") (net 1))
 (via (at 99.54242 47.159507) (size 0.6) (drill 0.3) (layers "F.Cu" "B.Cu") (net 1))
 (segment (start 103.25 54.925) (end 103.25 52.845) (width 0.25) (layer "B.Cu") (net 1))
 (segment (start 103.25 52.845) (end 104.133 51.962) (width 0.25) (layer "B.Cu") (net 1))
 (segment (start 93.607 51.67) (end 97.642554 51.67) (width 0.55) (layer "F.Cu") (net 2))
 (segment (start 97.642554 51.67) (end 99.797554 53.825) (width 0.55) (layer "F.Cu") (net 2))
 (segment (start 99.797554 53.825) (end 103.25 53.825) (width 0.55) (layer "F.Cu") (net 2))
 (segment (start 97.9 51.67) (end 98.949 50.621) (width 0.25) (layer "B.Cu") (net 6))
 (segment (start 93.607 51.67) (end 97.9 51.67) (width 0.25) (layer "B.Cu") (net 6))
 (segment (start 98.949 50.621) (end 98.949 48.232) (width 0.25) (layer "B.Cu") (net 6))
 (segment (start 98.949 48.232) (end 97.542 46.825) (width 0.25) (layer "B.Cu") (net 6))
 (segment (start 93.607 50.67) (end 94.452 49.825) (width 0.25) (layer "B.Cu") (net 5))
 (segment (start 94.452 49.825) (end 96.75 49.825) (width 0.25) (layer "B.Cu") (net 5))
 (segment (start 93.607 52.67) (end 95.595 52.67) (width 0.55) (layer "B.Cu") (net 7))
 (segment (start 95.595 52.67) (end 96.75 53.825) (width 0.55) (layer "B.Cu") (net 7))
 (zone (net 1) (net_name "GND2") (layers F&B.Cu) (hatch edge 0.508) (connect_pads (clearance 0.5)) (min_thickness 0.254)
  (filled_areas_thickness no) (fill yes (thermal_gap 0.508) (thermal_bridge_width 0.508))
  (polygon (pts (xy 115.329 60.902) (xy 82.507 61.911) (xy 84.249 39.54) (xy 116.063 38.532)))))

